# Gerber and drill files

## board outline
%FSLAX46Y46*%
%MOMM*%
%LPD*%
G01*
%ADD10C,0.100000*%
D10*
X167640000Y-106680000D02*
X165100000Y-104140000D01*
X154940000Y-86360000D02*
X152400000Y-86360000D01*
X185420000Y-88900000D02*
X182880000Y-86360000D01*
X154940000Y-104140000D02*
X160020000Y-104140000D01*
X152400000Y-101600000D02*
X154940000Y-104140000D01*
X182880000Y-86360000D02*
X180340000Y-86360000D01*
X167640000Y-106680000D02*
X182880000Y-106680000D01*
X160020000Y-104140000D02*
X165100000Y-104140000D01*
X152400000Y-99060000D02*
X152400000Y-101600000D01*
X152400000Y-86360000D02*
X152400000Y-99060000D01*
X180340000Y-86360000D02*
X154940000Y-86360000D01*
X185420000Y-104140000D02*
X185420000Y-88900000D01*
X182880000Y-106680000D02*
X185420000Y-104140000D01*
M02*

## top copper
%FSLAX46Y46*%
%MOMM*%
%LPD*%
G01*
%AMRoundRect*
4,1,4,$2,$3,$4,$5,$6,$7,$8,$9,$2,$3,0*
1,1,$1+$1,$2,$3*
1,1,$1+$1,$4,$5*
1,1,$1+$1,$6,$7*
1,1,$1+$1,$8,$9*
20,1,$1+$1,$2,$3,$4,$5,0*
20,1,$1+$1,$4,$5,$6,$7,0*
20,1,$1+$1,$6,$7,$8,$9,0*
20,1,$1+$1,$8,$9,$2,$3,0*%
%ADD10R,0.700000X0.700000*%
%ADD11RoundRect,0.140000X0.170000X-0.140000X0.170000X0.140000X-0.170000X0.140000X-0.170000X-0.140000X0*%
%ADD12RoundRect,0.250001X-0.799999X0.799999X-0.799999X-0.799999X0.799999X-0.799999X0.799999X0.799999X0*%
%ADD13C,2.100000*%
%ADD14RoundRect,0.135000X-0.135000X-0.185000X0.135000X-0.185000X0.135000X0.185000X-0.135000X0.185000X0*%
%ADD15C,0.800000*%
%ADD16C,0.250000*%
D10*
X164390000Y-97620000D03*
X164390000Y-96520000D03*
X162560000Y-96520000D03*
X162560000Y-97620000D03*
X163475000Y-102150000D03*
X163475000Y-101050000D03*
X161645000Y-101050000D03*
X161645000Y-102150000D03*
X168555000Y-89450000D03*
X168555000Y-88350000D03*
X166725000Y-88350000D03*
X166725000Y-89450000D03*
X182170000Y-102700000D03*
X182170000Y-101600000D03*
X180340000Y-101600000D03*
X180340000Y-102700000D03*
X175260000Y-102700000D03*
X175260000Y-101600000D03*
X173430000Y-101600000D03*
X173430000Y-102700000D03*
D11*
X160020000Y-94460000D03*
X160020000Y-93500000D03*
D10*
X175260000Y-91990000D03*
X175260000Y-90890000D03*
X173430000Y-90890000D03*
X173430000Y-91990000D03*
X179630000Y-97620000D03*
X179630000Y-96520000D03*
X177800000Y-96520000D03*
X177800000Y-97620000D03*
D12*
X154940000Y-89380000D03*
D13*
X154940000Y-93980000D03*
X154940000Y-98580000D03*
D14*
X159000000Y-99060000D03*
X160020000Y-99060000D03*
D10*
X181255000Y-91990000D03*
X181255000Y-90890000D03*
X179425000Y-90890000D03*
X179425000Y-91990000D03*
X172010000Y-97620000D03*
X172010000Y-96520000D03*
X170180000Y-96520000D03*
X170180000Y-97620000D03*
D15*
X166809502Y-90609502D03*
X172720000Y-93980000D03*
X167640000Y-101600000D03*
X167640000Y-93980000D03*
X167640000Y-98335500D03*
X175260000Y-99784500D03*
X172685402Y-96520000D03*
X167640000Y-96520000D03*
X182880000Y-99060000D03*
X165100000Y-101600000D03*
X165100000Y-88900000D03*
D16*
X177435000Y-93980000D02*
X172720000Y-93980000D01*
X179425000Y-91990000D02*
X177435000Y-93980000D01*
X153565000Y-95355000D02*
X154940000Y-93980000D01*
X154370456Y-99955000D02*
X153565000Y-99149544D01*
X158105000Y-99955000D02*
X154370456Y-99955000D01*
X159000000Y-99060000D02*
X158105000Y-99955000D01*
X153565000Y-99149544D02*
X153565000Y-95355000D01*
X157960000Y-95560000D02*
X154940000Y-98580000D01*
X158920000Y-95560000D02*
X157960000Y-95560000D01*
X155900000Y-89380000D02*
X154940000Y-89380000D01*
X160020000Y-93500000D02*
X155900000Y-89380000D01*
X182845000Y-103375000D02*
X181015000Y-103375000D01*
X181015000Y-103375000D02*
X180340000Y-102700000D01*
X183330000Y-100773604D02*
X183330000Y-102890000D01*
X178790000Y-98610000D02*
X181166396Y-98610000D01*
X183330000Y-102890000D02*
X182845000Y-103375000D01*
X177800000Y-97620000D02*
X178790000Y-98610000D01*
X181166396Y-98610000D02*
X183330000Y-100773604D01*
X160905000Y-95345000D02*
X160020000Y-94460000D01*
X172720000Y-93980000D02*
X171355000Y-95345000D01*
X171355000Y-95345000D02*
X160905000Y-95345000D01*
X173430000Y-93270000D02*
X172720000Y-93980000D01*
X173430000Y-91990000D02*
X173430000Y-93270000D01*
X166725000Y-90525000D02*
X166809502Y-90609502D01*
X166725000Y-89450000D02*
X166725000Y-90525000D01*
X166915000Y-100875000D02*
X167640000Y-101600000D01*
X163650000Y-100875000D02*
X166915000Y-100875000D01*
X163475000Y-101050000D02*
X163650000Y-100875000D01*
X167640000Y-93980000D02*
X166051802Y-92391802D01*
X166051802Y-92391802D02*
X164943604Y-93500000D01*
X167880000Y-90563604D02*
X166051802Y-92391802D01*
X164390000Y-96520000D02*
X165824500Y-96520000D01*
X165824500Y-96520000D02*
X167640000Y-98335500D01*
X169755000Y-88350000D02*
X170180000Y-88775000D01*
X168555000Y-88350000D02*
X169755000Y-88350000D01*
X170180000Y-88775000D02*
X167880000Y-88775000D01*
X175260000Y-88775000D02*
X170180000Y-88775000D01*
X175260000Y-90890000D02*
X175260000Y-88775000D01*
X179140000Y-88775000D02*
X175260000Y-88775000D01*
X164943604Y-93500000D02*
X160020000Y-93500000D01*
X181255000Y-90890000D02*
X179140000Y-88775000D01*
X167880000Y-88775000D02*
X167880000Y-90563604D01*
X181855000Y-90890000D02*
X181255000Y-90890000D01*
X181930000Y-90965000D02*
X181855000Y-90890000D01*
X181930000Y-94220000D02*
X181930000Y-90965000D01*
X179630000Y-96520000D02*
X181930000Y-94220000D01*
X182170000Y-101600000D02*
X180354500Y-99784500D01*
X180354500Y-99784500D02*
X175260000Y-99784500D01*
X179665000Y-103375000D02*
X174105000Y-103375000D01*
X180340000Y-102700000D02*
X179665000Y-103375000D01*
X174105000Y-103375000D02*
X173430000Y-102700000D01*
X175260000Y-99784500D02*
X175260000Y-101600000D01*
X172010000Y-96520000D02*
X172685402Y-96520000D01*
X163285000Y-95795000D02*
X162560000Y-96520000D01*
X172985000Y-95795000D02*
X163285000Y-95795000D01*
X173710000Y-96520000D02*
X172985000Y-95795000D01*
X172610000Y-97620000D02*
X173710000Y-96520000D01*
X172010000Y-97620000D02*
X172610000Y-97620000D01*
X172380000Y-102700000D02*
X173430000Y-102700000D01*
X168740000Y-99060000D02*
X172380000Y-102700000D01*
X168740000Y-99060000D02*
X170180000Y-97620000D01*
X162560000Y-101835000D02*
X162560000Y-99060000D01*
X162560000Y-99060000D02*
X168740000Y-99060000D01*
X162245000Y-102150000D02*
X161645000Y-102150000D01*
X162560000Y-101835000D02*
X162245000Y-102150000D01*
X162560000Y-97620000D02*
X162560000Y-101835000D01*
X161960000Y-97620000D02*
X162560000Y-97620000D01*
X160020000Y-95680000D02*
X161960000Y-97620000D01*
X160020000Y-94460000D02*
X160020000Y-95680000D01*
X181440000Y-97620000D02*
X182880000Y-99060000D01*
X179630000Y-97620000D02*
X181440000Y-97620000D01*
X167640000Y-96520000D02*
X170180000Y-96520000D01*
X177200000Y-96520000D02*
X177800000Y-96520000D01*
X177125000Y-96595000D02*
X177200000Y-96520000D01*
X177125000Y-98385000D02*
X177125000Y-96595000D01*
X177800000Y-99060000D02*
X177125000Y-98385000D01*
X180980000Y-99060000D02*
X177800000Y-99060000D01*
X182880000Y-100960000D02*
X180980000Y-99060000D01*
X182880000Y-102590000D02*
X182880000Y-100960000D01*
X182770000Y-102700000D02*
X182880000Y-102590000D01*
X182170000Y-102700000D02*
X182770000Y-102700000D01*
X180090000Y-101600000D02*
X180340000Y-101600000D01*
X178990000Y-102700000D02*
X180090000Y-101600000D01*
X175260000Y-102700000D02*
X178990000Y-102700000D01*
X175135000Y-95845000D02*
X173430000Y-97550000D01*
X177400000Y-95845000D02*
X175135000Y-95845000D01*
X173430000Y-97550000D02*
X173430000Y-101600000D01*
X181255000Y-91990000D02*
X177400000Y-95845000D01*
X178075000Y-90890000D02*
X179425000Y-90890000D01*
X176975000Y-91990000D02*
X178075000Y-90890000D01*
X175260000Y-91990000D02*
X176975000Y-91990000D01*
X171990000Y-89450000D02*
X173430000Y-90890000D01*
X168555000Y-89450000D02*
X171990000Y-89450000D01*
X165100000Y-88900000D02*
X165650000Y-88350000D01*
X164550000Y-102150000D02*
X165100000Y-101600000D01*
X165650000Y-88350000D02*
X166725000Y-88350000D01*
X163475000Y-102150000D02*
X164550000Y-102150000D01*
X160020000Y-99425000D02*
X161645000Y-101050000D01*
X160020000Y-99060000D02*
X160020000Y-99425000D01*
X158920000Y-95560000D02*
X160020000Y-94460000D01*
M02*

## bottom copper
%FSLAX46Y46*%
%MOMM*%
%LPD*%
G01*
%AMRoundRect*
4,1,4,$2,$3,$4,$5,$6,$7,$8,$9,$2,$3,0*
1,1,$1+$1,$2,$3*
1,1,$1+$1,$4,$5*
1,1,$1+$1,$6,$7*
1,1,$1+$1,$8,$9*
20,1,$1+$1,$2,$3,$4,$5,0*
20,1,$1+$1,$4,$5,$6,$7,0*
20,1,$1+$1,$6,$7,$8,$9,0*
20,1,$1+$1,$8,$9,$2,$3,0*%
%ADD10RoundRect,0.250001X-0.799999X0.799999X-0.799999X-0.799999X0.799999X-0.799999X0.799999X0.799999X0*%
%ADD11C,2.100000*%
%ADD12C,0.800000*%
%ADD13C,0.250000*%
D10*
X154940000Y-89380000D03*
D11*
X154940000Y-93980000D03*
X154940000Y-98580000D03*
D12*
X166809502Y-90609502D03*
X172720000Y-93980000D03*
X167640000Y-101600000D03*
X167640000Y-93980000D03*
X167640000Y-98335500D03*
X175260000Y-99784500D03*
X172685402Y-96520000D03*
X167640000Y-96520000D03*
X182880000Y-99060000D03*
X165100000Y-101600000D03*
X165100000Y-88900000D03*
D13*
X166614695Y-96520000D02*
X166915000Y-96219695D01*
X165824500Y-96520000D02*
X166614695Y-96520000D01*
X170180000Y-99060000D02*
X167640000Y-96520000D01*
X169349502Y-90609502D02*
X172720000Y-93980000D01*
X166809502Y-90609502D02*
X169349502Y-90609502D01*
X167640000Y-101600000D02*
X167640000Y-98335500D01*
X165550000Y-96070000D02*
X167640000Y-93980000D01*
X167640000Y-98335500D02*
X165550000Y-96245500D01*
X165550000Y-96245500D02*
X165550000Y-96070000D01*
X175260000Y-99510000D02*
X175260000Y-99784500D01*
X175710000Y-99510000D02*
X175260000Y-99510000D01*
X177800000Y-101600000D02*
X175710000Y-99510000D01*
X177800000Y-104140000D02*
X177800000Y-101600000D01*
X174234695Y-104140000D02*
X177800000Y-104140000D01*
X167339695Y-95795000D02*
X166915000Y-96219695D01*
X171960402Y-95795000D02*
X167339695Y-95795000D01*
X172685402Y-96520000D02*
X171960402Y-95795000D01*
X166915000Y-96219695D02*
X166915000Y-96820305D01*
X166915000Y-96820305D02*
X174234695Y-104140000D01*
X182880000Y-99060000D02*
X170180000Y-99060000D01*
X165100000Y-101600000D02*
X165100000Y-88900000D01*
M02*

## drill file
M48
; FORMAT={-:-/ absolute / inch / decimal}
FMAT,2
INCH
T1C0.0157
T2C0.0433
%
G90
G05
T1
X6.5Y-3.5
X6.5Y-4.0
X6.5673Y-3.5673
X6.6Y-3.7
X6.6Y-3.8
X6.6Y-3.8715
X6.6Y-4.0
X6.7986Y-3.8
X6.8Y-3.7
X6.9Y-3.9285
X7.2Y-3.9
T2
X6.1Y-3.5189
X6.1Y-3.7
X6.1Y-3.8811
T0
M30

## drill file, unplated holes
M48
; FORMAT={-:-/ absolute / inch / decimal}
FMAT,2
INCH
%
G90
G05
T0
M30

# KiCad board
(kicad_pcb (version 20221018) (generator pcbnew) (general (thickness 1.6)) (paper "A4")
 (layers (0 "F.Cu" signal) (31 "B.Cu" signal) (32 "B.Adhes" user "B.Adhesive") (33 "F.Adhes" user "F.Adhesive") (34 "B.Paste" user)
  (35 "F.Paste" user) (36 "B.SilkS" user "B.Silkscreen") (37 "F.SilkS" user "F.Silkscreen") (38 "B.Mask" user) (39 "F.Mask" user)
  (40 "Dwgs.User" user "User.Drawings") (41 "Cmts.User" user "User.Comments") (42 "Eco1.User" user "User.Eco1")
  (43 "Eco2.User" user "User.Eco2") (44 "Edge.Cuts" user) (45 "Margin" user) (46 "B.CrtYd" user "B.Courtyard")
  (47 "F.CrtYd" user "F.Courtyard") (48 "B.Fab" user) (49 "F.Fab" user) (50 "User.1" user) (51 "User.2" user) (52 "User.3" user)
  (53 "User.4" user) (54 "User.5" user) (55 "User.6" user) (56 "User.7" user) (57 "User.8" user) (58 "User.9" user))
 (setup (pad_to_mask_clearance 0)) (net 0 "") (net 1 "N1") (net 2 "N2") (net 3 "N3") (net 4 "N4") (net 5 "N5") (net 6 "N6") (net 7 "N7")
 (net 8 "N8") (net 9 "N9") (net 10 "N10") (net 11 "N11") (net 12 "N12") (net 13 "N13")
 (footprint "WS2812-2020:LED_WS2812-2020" (layer "F.Cu") (at 163.475 97.07)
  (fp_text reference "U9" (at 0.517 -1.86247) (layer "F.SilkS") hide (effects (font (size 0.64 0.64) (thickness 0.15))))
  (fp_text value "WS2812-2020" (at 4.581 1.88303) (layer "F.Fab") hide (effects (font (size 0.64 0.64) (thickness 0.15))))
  (pad "1" smd rect (at 0.915 0.55) (size 0.7 0.7) (layers "F.Cu" "F.Paste" "F.Mask") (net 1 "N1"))
  (pad "2" smd rect (at 0.915 -0.55) (size 0.7 0.7) (layers "F.Cu" "F.Paste" "F.Mask") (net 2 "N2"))
  (pad "3" smd rect (at -0.915 -0.55) (size 0.7 0.7) (layers "F.Cu" "F.Paste" "F.Mask") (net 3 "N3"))
  (pad "4" smd rect (at -0.915 0.55) (size 0.7 0.7) (layers "F.Cu" "F.Paste" "F.Mask") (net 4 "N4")))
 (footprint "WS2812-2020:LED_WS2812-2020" (layer "F.Cu") (at 162.56 101.6)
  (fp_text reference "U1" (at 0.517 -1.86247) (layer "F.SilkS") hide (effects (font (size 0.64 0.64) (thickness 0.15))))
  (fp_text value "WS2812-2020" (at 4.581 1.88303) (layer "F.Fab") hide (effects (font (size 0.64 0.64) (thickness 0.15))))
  (pad "1" smd rect (at 0.915 0.55) (size 0.7 0.7) (layers "F.Cu" "F.Paste" "F.Mask") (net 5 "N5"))
  (pad "2" smd rect (at 0.915 -0.55) (size 0.7 0.7) (layers "F.Cu" "F.Paste" "F.Mask") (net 2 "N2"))
  (pad "3" smd rect (at -0.915 -0.55) (size 0.7 0.7) (layers "F.Cu" "F.Paste" "F.Mask") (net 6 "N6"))
  (pad "4" smd rect (at -0.915 0.55) (size 0.7 0.7) (layers "F.Cu" "F.Paste" "F.Mask") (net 4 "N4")))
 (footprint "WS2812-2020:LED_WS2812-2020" (layer "F.Cu") (at 167.64 88.9)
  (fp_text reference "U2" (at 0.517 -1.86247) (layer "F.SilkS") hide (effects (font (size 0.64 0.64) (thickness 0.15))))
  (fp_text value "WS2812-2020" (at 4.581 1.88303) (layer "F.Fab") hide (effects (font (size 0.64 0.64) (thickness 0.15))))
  (pad "1" smd rect (at 0.915 0.55) (size 0.7 0.7) (layers "F.Cu" "F.Paste" "F.Mask") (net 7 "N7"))
  (pad "2" smd rect (at 0.915 -0.55) (size 0.7 0.7) (layers "F.Cu" "F.Paste" "F.Mask") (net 2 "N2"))
  (pad "3" smd rect (at -0.915 -0.55) (size 0.7 0.7) (layers "F.Cu" "F.Paste" "F.Mask") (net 5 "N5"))
  (pad "4" smd rect (at -0.915 0.55) (size 0.7 0.7) (layers "F.Cu" "F.Paste" "F.Mask") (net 4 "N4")))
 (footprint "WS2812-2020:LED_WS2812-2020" (layer "F.Cu") (at 181.255 102.15)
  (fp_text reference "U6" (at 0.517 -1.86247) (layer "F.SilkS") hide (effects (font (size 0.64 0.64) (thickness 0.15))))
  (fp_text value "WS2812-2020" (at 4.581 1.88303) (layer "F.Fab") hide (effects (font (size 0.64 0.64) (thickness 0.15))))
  (pad "1" smd rect (at 0.915 0.55) (size 0.7 0.7) (layers "F.Cu" "F.Paste" "F.Mask") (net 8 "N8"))
  (pad "2" smd rect (at 0.915 -0.55) (size 0.7 0.7) (layers "F.Cu" "F.Paste" "F.Mask") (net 2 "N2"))
  (pad "3" smd rect (at -0.915 -0.55) (size 0.7 0.7) (layers "F.Cu" "F.Paste" "F.Mask") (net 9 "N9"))
  (pad "4" smd rect (at -0.915 0.55) (size 0.7 0.7) (layers "F.Cu" "F.Paste" "F.Mask") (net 4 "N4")))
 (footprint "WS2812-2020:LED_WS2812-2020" (layer "F.Cu") (at 174.345 102.15)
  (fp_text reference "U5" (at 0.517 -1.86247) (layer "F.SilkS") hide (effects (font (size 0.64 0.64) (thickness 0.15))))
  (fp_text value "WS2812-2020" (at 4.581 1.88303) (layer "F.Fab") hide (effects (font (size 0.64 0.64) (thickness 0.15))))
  (pad "1" smd rect (at 0.915 0.55) (size 0.7 0.7) (layers "F.Cu" "F.Paste" "F.Mask") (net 9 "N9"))
  (pad "2" smd rect (at 0.915 -0.55) (size 0.7 0.7) (layers "F.Cu" "F.Paste" "F.Mask") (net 2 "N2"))
  (pad "3" smd rect (at -0.915 -0.55) (size 0.7 0.7) (layers "F.Cu" "F.Paste" "F.Mask") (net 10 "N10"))
  (pad "4" smd rect (at -0.915 0.55) (size 0.7 0.7) (layers "F.Cu" "F.Paste" "F.Mask") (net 4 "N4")))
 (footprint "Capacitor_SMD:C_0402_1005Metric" (layer "F.Cu") (at 160.02 93.98 90)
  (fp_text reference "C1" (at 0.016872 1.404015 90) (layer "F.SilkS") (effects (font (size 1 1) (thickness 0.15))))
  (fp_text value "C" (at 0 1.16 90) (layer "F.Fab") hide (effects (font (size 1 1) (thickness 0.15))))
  (pad "1" smd roundrect (at -0.48 0 90) (size 0.56 0.62) (layers "F.Cu" "F.Paste" "F.Mask") (roundrect_rratio 0.25) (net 4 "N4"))
  (pad "2" smd roundrect (at 0.48 0 90) (size 0.56 0.62) (layers "F.Cu" "F.Paste" "F.Mask") (roundrect_rratio 0.25) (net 2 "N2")))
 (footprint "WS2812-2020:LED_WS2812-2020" (layer "F.Cu") (at 174.345 91.44)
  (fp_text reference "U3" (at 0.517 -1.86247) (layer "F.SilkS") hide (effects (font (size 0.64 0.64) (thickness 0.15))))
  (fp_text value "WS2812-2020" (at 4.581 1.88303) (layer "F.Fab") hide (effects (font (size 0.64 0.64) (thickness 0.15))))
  (pad "1" smd rect (at 0.915 0.55) (size 0.7 0.7) (layers "F.Cu" "F.Paste" "F.Mask") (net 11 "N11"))
  (pad "2" smd rect (at 0.915 -0.55) (size 0.7 0.7) (layers "F.Cu" "F.Paste" "F.Mask") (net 2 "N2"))
  (pad "3" smd rect (at -0.915 -0.55) (size 0.7 0.7) (layers "F.Cu" "F.Paste" "F.Mask") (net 7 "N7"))
  (pad "4" smd rect (at -0.915 0.55) (size 0.7 0.7) (layers "F.Cu" "F.Paste" "F.Mask") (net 4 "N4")))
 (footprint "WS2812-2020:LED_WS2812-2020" (layer "F.Cu") (at 178.715 97.07)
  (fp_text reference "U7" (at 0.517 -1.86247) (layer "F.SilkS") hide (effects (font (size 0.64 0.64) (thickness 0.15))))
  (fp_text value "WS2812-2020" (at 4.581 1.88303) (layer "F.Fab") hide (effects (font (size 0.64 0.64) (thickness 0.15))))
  (pad "1" smd rect (at 0.915 0.55) (size 0.7 0.7) (layers "F.Cu" "F.Paste" "F.Mask") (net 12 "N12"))
  (pad "2" smd rect (at 0.915 -0.55) (size 0.7 0.7) (layers "F.Cu" "F.Paste" "F.Mask") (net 2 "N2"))
  (pad "3" smd rect (at -0.915 -0.55) (size 0.7 0.7) (layers "F.Cu" "F.Paste" "F.Mask") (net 8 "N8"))
  (pad "4" smd rect (at -0.915 0.55) (size 0.7 0.7) (layers "F.Cu" "F.Paste" "F.Mask") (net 4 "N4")))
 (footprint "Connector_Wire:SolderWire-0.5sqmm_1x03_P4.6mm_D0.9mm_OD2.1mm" (layer "F.Cu") (at 154.94 89.38 -90)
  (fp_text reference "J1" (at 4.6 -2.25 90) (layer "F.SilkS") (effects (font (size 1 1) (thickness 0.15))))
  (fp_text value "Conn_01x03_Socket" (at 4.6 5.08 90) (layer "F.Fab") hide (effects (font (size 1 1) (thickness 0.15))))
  (pad "1" thru_hole roundrect (at 0 0 270) (size 2.1 2.1) (drill 1.1) (layers "*.Cu" "*.Mask") (roundrect_rratio 0.1190480952) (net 2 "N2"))
  (pad "2" thru_hole circle (at 4.6 0 270) (size 2.1 2.1) (drill 1.1) (layers "*.Cu" "*.Mask") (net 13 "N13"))
  (pad "3" thru_hole circle (at 9.2 0 270) (size 2.1 2.1) (drill 1.1) (layers "*.Cu" "*.Mask") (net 4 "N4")))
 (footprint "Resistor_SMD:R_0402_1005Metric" (layer "F.Cu") (at 159.51 99.06)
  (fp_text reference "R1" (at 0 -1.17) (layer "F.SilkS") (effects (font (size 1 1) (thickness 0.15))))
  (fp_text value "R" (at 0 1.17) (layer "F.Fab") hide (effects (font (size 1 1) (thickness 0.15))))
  (pad "1" smd roundrect (at -0.51 0) (size 0.54 0.64) (layers "F.Cu" "F.Paste" "F.Mask") (roundrect_rratio 0.25) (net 13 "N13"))
  (pad "2" smd roundrect (at 0.51 0) (size 0.54 0.64) (layers "F.Cu" "F.Paste" "F.Mask") (roundrect_rratio 0.25) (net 6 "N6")))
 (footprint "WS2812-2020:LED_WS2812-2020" (layer "F.Cu") (at 180.34 91.44)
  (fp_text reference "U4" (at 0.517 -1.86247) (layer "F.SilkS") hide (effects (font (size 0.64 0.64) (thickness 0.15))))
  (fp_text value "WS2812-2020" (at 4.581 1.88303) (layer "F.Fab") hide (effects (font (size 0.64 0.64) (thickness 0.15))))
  (pad "1" smd rect (at 0.915 0.55) (size 0.7 0.7) (layers "F.Cu" "F.Paste" "F.Mask") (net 10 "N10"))
  (pad "2" smd rect (at 0.915 -0.55) (size 0.7 0.7) (layers "F.Cu" "F.Paste" "F.Mask") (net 2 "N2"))
  (pad "3" smd rect (at -0.915 -0.55) (size 0.7 0.7) (layers "F.Cu" "F.Paste" "F.Mask") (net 11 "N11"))
  (pad "4" smd rect (at -0.915 0.55) (size 0.7 0.7) (layers "F.Cu" "F.Paste" "F.Mask") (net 4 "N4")))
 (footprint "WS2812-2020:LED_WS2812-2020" (layer "F.Cu") (at 171.095 97.07)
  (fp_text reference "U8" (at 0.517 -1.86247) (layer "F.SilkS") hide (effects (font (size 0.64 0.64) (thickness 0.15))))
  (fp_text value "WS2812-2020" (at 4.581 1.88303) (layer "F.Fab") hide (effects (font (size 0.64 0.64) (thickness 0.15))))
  (pad "1" smd rect (at 0.915 0.55) (size 0.7 0.7) (layers "F.Cu" "F.Paste" "F.Mask") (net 3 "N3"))
  (pad "2" smd rect (at 0.915 -0.55) (size 0.7 0.7) (layers "F.Cu" "F.Paste" "F.Mask") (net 2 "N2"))
  (pad "3" smd rect (at -0.915 -0.55) (size 0.7 0.7) (layers "F.Cu" "F.Paste" "F.Mask") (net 12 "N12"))
  (pad "4" smd rect (at -0.915 0.55) (size 0.7 0.7) (layers "F.Cu" "F.Paste" "F.Mask") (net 4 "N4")))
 (gr_line (start 182.88 106.68) (end 185.42 106.68) (stroke (width 0.1) (type default)) (layer "Edge.Cuts"))
 (gr_line (start 167.64 106.68) (end 165.1 106.68) (stroke (width 0.1) (type default)) (layer "Edge.Cuts"))
 (gr_line (start 185.42 86.36) (end 182.88 86.36) (stroke (width 0.1) (type default)) (layer "Edge.Cuts"))
 (gr_line (start 160.02 106.68) (end 165.1 106.68) (stroke (width 0.1) (type default)) (layer "Edge.Cuts"))
 (gr_line (start 180.34 86.36) (end 154.94 86.36) (stroke (width 0.1) (type default)) (layer "Edge.Cuts"))
 (gr_line (start 152.4 106.68) (end 160.02 106.68) (stroke (width 0.1) (type default)) (layer "Edge.Cuts"))
 (gr_line (start 185.42 88.9) (end 185.42 86.36) (stroke (width 0.1) (type default)) (layer "Edge.Cuts"))
 (gr_line (start 152.4 86.36) (end 152.4 99.06) (stroke (width 0.1) (type default)) (layer "Edge.Cuts"))
 (gr_line (start 152.4 101.6) (end 152.4 106.68) (stroke (width 0.1) (type default)) (layer "Edge.Cuts"))
 (gr_line (start 185.42 104.14) (end 185.42 88.9) (stroke (width 0.1) (type default)) (layer "Edge.Cuts"))
 (gr_line (start 182.88 86.36) (end 180.34 86.36) (stroke (width 0.1) (type default)) (layer "Edge.Cuts"))
 (gr_line (start 154.94 86.36) (end 152.4 86.36) (stroke (width 0.1) (type default)) (layer "Edge.Cuts"))
 (gr_line (start 167.64 106.68) (end 182.88 106.68) (stroke (width 0.1) (type default)) (layer "Edge.Cuts"))
 (gr_line (start 185.42 106.68) (end 185.42 104.14) (stroke (width 0.1) (type default)) (layer "Edge.Cuts"))
 (gr_line (start 152.4 99.06) (end 152.4 101.6) (stroke (width 0.1) (type default)) (layer "Edge.Cuts"))
 (segment (start 160.02 95.68) (end 161.96 97.62) (width 0.25) (layer "F.Cu") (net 4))
 (segment (start 181.166396 98.61) (end 183.33 100.773604) (width 0.25) (layer "F.Cu") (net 4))
 (segment (start 162.56 101.835) (end 162.245 102.15) (width 0.25) (layer "F.Cu") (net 4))
 (segment (start 160.02 94.46) (end 160.02 95.68) (width 0.25) (layer "F.Cu") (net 4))
 (segment (start 168.74 99.06) (end 170.18 97.62) (width 0.25) (layer "F.Cu") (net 4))
 (segment (start 181.015 103.375) (end 180.34 102.7) (width 0.25) (layer "F.Cu") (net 4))
 (segment (start 161.96 97.62) (end 162.56 97.62) (width 0.25) (layer "F.Cu") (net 4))
 (segment (start 180.34 102.7) (end 179.665 103.375) (width 0.25) (layer "F.Cu") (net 4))
 (segment (start 183.33 102.89) (end 182.845 103.375) (width 0.25) (layer "F.Cu") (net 4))
 (segment (start 177.435 93.98) (end 172.72 93.98) (width 0.25) (layer "F.Cu") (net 4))
 (segment (start 172.38 102.7) (end 173.43 102.7) (width 0.25) (layer "F.Cu") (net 4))
 (segment (start 172.72 93.98) (end 171.355 95.345) (width 0.25) (layer "F.Cu") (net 4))
 (segment (start 171.355 95.345) (end 160.905 95.345) (width 0.25) (layer "F.Cu") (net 4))
 (segment (start 173.43 93.27) (end 172.72 93.98) (width 0.25) (layer "F.Cu") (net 4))
 (segment (start 183.33 100.773604) (end 183.33 102.89) (width 0.25) (layer "F.Cu") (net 4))
 (segment (start 173.43 91.99) (end 173.43 93.27) (width 0.25) (layer "F.Cu") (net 4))
 (segment (start 178.79 98.61) (end 181.166396 98.61) (width 0.25) (layer "F.Cu") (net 4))
 (segment (start 158.92 95.56) (end 157.96 95.56) (width 0.25) (layer "F.Cu") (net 4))
 (segment (start 158.92 95.56) (end 160.02 94.46) (width 0.25) (layer "F.Cu") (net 4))
 (segment (start 168.74 99.06) (end 172.38 102.7) (width 0.25) (layer "F.Cu") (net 4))
 (segment (start 166.725 90.525) (end 166.809502 90.609502) (width 0.25) (layer "F.Cu") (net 4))
 (segment (start 157.96 95.56) (end 154.94 98.58) (width 0.25) (layer "F.Cu") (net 4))
 (segment (start 177.8 97.62) (end 178.79 98.61) (width 0.25) (layer "F.Cu") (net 4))
 (segment (start 166.725 89.45) (end 166.725 90.525) (width 0.25) (layer "F.Cu") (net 4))
 (segment (start 179.425 91.99) (end 177.435 93.98) (width 0.25) (layer "F.Cu") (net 4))
 (segment (start 162.56 101.835) (end 162.56 99.06) (width 0.25) (layer "F.Cu") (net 4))
 (segment (start 182.845 103.375) (end 181.015 103.375) (width 0.25) (layer "F.Cu") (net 4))
 (segment (start 160.905 95.345) (end 160.02 94.46) (width 0.25) (layer "F.Cu") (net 4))
 (segment (start 162.56 99.06) (end 168.74 99.06) (width 0.25) (layer "F.Cu") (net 4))
 (segment (start 174.105 103.375) (end 173.43 102.7) (width 0.25) (layer "F.Cu") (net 4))
 (segment (start 162.56 97.62) (end 162.56 101.835) (width 0.25) (layer "F.Cu") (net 4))
 (segment (start 179.665 103.375) (end 174.105 103.375) (width 0.25) (layer "F.Cu") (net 4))
 (segment (start 162.245 102.15) (end 161.645 102.15) (width 0.25) (layer "F.Cu") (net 4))
 (via (at 166.809502 90.609502) (size 0.8) (drill 0.4) (layers "F.Cu" "B.Cu") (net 4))
 (via (at 172.72 93.98) (size 0.8) (drill 0.4) (layers "F.Cu" "B.Cu") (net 4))
 (segment (start 169.349502 90.609502) (end 172.72 93.98) (width 0.25) (layer "B.Cu") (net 4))
 (segment (start 166.809502 90.609502) (end 169.349502 90.609502) (width 0.25) (layer "B.Cu") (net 4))
 (segment (start 160.02 93.5) (end 155.9 89.38) (width 0.25) (layer "F.Cu") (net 2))
 (segment (start 182.17 101.6) (end 180.3545 99.7845) (width 0.25) (layer "F.Cu") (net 2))
 (segment (start 175.26 90.89) (end 175.26 88.775) (width 0.25) (layer "F.Cu") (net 2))
 (segment (start 166.051802 92.391802) (end 164.943604 93.5) (width 0.25) (layer "F.Cu") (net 2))
 (segment (start 172.01 96.52) (end 172.685402 96.52) (width 0.25) (layer "F.Cu") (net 2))
 (segment (start 164.39 96.52) (end 165.8245 96.52) (width 0.25) (layer "F.Cu") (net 2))
 (segment (start 180.3545 99.7845) (end 175.26 99.7845) (width 0.25) (layer "F.Cu") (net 2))
 (segment (start 165.8245 96.52) (end 167.64 98.3355) (width 0.25) (layer "F.Cu") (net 2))
 (segment (start 181.255 90.89) (end 179.14 88.775) (width 0.25) (layer "F.Cu") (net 2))
 (segment (start 167.64 93.98) (end 166.051802 92.391802) (width 0.25) (layer "F.Cu") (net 2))
 (segment (start 179.63 96.52) (end 181.93 94.22) (width 0.25) (layer "F.Cu") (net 2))
 (segment (start 163.475 101.05) (end 163.65 100.875) (width 0.25) (layer "F.Cu") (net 2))
 (segment (start 170.18 88.775) (end 167.88 88.775) (width 0.25) (layer "F.Cu") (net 2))
 (segment (start 179.14 88.775) (end 175.26 88.775) (width 0.25) (layer "F.Cu") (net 2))
 (segment (start 175.26 88.775) (end 170.18 88.775) (width 0.25) (layer "F.Cu") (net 2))
 (segment (start 175.26 99.7845) (end 175.26 101.6) (width 0.25) (layer "F.Cu") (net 2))
 (segment (start 168.555 88.35) (end 169.755 88.35) (width 0.25) (layer "F.Cu") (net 2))
 (segment (start 163.65 100.875) (end 166.915 100.875) (width 0.25) (layer "F.Cu") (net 2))
 (segment (start 169.755 88.35) (end 170.18 88.775) (width 0.25) (layer "F.Cu") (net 2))
 (segment (start 166.915 100.875) (end 167.64 101.6) (width 0.25) (layer "F.Cu") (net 2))
 (segment (start 181.93 94.22) (end 181.93 90.965) (width 0.25) (layer "F.Cu") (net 2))
 (segment (start 167.88 88.775) (end 167.88 90.563604) (width 0.25) (layer "F.Cu") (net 2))
 (segment (start 164.943604 93.5) (end 160.02 93.5) (width 0.25) (layer "F.Cu") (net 2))
 (segment (start 167.88 90.563604) (end 166.051802 92.391802) (width 0.25) (layer "F.Cu") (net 2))
 (segment (start 155.9 89.38) (end 154.94 89.38) (width 0.25) (layer "F.Cu") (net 2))
 (segment (start 181.93 90.965) (end 181.855 90.89) (width 0.25) (layer "F.Cu") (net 2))
 (segment (start 181.855 90.89) (end 181.255 90.89) (width 0.25) (layer "F.Cu") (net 2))
 (via (at 172.685402 96.52) (size 0.8) (drill 0.4) (layers "F.Cu" "B.Cu") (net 2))
 (via (at 167.64 101.6) (size 0.8) (drill 0.4) (layers "F.Cu" "B.Cu") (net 2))
 (via (at 167.64 93.98) (size 0.8) (drill 0.4) (layers "F.Cu" "B.Cu") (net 2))
 (via (at 167.64 98.3355) (size 0.8) (drill 0.4) (layers "F.Cu" "B.Cu") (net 2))
 (via (at 175.26 99.7845) (size 0.8) (drill 0.4) (layers "F.Cu" "B.Cu") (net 2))
 (segment (start 175.71 99.51) (end 175.26 99.51) (width 0.25) (layer "B.Cu") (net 2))
 (segment (start 172.685402 96.52) (end 171.960402 95.795) (width 0.25) (layer "B.Cu") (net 2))
 (segment (start 167.64 101.6) (end 167.64 98.3355) (width 0.25) (layer "B.Cu") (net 2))
 (segment (start 166.915 96.219695) (end 166.915 96.820305) (width 0.25) (layer "B.Cu") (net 2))
 (segment (start 167.339695 95.795) (end 166.915 96.219695) (width 0.25) (layer "B.Cu") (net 2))
 (segment (start 165.8245 96.52) (end 166.614695 96.52) (width 0.25) (layer "B.Cu") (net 2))
 (segment (start 177.8 101.6) (end 175.71 99.51) (width 0.25) (layer "B.Cu") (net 2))
 (segment (start 167.64 98.3355) (end 165.55 96.2455) (width 0.25) (layer "B.Cu") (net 2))
 (segment (start 165.55 96.2455) (end 165.55 96.07) (width 0.25) (layer "B.Cu") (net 2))
 (segment (start 174.234695 104.14) (end 177.8 104.14) (width 0.25) (layer "B.Cu") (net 2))
 (segment (start 166.915 96.820305) (end 174.234695 104.14) (width 0.25) (layer "B.Cu") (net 2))
 (segment (start 171.960402 95.795) (end 167.339695 95.795) (width 0.25) (layer "B.Cu") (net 2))
 (segment (start 165.55 96.07) (end 167.64 93.98) (width 0.25) (layer "B.Cu") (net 2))
 (segment (start 177.8 104.14) (end 177.8 101.6) (width 0.25) (layer "B.Cu") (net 2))
 (segment (start 166.614695 96.52) (end 166.915 96.219695) (width 0.25) (layer "B.Cu") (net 2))
 (segment (start 175.26 99.51) (end 175.26 99.7845) (width 0.25) (layer "B.Cu") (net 2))
 (segment (start 153.565 99.149544) (end 153.565 95.355) (width 0.25) (layer "F.Cu") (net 13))
 (segment (start 158.105 99.955) (end 154.370456 99.955) (width 0.25) (layer "F.Cu") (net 13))
 (segment (start 159 99.06) (end 158.105 99.955) (width 0.25) (layer "F.Cu") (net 13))
 (segment (start 153.565 95.355) (end 154.94 93.98) (width 0.25) (layer "F.Cu") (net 13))
 (segment (start 154.370456 99.955) (end 153.565 99.149544) (width 0.25) (layer "F.Cu") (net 13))
 (segment (start 160.02 99.425) (end 161.645 101.05) (width 0.25) (layer "F.Cu") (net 6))
 (segment (start 160.02 99.06) (end 160.02 99.425) (width 0.25) (layer "F.Cu") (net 6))
 (segment (start 164.55 102.15) (end 165.1 101.6) (width 0.25) (layer "F.Cu") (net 5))
 (segment (start 165.65 88.35) (end 166.725 88.35) (width 0.25) (layer "F.Cu") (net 5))
 (segment (start 163.475 102.15) (end 164.55 102.15) (width 0.25) (layer "F.Cu") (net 5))
 (segment (start 165.1 88.9) (end 165.65 88.35) (width 0.25) (layer "F.Cu") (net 5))
 (via (at 165.1 88.9) (size 0.8) (drill 0.4) (layers "F.Cu" "B.Cu") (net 5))
 (via (at 165.1 101.6) (size 0.8) (drill 0.4) (layers "F.Cu" "B.Cu") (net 5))
 (segment (start 165.1 101.6) (end 165.1 88.9) (width 0.25) (layer "B.Cu") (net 5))
 (segment (start 171.99 89.45) (end 173.43 90.89) (width 0.25) (layer "F.Cu") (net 7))
 (segment (start 168.555 89.45) (end 171.99 89.45) (width 0.25) (layer "F.Cu") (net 7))
 (segment (start 178.075 90.89) (end 179.425 90.89) (width 0.25) (layer "F.Cu") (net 11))
 (segment (start 176.975 91.99) (end 178.075 90.89) (width 0.25) (layer "F.Cu") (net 11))
 (segment (start 175.26 91.99) (end 176.975 91.99) (width 0.25) (layer "F.Cu") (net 11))
 (segment (start 177.4 95.845) (end 175.135 95.845) (width 0.25) (layer "F.Cu") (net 10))
 (segment (start 173.43 97.55) (end 173.43 101.6) (width 0.25) (layer "F.Cu") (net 10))
 (segment (start 175.135 95.845) (end 173.43 97.55) (width 0.25) (layer "F.Cu") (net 10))
 (segment (start 181.255 91.99) (end 177.4 95.845) (width 0.25) (layer "F.Cu") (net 10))
 (segment (start 180.09 101.6) (end 180.34 101.6) (width 0.25) (layer "F.Cu") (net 9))
 (segment (start 178.99 102.7) (end 180.09 101.6) (width 0.25) (layer "F.Cu") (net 9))
 (segment (start 175.26 102.7) (end 178.99 102.7) (width 0.25) (layer "F.Cu") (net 9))
 (segment (start 182.77 102.7) (end 182.88 102.59) (width 0.25) (layer "F.Cu") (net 8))
 (segment (start 182.17 102.7) (end 182.77 102.7) (width 0.25) (layer "F.Cu") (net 8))
 (segment (start 182.88 102.59) (end 182.88 100.96) (width 0.25) (layer "F.Cu") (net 8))
 (segment (start 180.98 99.06) (end 177.8 99.06) (width 0.25) (layer "F.Cu") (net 8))
 (segment (start 177.8 99.06) (end 177.125 98.385) (width 0.25) (layer "F.Cu") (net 8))
 (segment (start 182.88 100.96) (end 180.98 99.06) (width 0.25) (layer "F.Cu") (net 8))
 (segment (start 177.125 96.595) (end 177.2 96.52) (width 0.25) (layer "F.Cu") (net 8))
 (segment (start 177.2 96.52) (end 177.8 96.52) (width 0.25) (layer "F.Cu") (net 8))
 (segment (start 177.125 98.385) (end 177.125 96.595) (width 0.25) (layer "F.Cu") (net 8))
 (segment (start 167.64 96.52) (end 170.18 96.52) (width 0.25) (layer "F.Cu") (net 12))
 (segment (start 181.44 97.62) (end 182.88 99.06) (width 0.25) (layer "F.Cu") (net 12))
 (segment (start 179.63 97.62) (end 181.44 97.62) (width 0.25) (layer "F.Cu") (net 12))
 (via (at 182.88 99.06) (size 0.8) (drill 0.4) (layers "F.Cu" "B.Cu") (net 12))
 (via (at 167.64 96.52) (size 0.8) (drill 0.4) (layers "F.Cu" "B.Cu") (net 12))
 (segment (start 182.88 99.06) (end 170.18 99.06) (width 0.25) (layer "B.Cu") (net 12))
 (segment (start 170.18 99.06) (end 167.64 96.52) (width 0.25) (layer "B.Cu") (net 12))
 (segment (start 172.61 97.62) (end 173.71 96.52) (width 0.25) (layer "F.Cu") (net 3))
 (segment (start 172.985 95.795) (end 163.285 95.795) (width 0.25) (layer "F.Cu") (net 3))
 (segment (start 163.285 95.795) (end 162.56 96.52) (width 0.25) (layer "F.Cu") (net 3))
 (segment (start 172.01 97.62) (end 172.61 97.62) (width 0.25) (layer "F.Cu") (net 3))
 (segment (start 173.71 96.52) (end 172.985 95.795) (width 0.25) (layer "F.Cu") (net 3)))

